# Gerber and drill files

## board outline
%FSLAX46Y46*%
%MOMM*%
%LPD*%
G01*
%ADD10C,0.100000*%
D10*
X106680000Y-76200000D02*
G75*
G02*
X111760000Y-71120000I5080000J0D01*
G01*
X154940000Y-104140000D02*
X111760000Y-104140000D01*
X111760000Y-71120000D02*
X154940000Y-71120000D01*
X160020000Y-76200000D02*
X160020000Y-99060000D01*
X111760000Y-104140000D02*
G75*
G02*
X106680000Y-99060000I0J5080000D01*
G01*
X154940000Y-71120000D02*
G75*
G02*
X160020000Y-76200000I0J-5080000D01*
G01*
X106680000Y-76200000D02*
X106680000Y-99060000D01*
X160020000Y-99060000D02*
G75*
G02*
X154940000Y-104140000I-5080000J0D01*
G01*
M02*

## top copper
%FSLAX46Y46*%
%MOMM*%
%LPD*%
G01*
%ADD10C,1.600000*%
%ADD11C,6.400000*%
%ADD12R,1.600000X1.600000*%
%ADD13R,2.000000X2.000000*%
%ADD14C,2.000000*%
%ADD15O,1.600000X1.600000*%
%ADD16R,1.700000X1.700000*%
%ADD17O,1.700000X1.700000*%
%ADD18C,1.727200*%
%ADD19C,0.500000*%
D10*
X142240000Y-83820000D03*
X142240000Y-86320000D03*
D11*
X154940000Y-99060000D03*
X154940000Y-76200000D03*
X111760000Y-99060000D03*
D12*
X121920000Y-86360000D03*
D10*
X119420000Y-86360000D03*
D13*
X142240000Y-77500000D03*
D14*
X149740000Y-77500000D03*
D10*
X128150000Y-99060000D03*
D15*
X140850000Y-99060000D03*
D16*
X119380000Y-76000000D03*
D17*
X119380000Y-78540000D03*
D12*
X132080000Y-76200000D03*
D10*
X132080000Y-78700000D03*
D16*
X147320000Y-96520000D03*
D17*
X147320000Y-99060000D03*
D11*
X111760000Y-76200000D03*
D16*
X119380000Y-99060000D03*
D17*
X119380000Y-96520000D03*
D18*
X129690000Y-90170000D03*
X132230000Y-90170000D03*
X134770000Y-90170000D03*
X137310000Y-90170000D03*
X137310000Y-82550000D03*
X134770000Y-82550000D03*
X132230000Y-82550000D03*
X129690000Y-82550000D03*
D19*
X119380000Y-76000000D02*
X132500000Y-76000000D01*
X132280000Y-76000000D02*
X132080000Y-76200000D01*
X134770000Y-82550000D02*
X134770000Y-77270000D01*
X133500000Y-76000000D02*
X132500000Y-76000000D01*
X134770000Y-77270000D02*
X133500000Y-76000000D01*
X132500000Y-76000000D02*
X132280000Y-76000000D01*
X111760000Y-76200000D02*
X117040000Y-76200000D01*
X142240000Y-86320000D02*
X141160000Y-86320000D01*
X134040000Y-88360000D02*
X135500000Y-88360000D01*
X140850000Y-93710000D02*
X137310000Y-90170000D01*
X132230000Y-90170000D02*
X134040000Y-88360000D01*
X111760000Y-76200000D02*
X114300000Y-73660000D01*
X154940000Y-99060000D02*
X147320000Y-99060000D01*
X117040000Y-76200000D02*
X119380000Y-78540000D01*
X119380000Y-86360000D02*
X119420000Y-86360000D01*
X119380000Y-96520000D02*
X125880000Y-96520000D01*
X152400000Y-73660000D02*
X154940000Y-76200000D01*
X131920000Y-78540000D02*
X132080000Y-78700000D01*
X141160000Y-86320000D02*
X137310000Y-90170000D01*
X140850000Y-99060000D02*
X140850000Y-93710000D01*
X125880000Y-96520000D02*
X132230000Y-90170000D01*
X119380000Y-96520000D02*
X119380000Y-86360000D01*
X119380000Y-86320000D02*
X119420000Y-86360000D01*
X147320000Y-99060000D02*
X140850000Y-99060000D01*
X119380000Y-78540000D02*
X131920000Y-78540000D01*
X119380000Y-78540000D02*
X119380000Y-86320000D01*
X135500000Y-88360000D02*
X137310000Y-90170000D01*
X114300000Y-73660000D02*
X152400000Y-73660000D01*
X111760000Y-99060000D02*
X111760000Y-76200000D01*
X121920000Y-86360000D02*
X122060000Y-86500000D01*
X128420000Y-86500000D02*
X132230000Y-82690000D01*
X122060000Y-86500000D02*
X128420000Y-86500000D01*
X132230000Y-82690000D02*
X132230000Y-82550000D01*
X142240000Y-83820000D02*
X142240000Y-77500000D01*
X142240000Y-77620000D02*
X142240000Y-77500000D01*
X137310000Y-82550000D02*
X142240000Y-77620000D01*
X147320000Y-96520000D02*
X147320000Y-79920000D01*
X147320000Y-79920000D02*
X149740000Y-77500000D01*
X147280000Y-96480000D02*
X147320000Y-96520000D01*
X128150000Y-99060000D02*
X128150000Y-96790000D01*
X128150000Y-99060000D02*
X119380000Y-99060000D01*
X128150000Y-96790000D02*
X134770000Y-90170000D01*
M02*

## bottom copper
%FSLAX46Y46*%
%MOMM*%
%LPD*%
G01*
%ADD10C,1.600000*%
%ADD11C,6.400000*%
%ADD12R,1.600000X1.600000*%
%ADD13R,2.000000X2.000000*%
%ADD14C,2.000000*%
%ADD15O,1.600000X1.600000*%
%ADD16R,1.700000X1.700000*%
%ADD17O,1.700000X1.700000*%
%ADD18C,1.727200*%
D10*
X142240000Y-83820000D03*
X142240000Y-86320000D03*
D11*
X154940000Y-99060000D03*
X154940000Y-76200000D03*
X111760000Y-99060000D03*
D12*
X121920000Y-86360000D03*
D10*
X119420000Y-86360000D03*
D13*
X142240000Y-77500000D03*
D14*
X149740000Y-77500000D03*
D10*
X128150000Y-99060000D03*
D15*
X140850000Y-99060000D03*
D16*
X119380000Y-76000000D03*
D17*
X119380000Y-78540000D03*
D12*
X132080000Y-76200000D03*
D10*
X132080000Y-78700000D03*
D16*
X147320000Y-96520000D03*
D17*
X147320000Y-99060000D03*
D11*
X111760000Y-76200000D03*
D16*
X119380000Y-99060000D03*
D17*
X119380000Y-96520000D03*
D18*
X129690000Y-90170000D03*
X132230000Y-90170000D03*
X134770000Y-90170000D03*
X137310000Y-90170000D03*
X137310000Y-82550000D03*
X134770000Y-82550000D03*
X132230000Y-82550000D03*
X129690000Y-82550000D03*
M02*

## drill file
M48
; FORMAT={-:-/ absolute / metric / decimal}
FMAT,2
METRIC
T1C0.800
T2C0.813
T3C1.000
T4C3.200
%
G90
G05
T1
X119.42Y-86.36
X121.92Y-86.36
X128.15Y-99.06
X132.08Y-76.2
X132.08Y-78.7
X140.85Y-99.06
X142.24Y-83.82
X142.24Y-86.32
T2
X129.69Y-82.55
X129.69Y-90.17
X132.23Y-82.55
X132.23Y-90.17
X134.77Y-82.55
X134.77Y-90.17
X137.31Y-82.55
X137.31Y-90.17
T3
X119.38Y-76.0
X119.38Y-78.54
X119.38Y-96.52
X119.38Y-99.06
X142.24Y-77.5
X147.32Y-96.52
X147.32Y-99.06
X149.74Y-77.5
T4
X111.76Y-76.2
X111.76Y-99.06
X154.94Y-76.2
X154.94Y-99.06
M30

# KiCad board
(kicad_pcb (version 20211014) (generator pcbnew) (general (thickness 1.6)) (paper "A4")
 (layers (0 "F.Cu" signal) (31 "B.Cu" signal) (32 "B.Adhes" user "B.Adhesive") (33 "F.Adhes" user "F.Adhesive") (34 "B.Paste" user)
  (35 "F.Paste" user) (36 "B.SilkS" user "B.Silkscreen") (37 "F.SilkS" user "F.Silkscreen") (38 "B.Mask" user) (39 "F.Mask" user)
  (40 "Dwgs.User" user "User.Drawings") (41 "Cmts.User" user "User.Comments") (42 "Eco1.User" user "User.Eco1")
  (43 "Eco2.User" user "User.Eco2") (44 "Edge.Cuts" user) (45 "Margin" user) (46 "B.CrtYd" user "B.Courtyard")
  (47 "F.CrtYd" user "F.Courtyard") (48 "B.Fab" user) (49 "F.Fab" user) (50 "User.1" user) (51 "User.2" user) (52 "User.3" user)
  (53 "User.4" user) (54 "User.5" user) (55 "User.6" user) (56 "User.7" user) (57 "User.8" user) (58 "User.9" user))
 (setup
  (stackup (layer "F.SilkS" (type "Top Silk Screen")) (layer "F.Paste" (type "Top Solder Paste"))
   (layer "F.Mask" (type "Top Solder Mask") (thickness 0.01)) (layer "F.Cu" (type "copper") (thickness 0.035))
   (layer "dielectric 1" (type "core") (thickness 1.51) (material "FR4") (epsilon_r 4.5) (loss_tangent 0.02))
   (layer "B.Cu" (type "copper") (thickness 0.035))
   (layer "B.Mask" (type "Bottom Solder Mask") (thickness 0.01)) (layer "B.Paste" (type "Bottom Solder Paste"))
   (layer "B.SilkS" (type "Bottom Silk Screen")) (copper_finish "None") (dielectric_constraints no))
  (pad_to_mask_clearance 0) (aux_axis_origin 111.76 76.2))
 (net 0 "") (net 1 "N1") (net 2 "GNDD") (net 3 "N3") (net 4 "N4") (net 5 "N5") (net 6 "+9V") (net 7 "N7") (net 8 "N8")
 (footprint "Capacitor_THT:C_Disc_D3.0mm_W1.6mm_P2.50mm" (layer "F.Cu") (at 142.24 83.82 -90)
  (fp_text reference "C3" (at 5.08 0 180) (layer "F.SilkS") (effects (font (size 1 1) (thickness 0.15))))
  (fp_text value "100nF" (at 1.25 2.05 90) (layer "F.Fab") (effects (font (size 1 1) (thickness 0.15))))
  (pad "1" thru_hole circle (at 0 0 270) (size 1.6 1.6) (drill 0.8) (layers *.Cu *.Mask) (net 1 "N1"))
  (pad "2" thru_hole circle (at 2.5 0 270) (size 1.6 1.6) (drill 0.8) (layers *.Cu *.Mask) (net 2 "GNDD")))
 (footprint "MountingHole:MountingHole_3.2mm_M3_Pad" (layer "F.Cu") (at 154.94 99.06)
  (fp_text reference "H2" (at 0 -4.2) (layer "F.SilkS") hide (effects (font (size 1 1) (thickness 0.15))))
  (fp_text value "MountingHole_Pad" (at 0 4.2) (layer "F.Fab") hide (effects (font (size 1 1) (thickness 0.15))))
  (pad "1" thru_hole circle (at 0 0) (size 6.4 6.4) (drill 3.2) (layers *.Cu *.Mask) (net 2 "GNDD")))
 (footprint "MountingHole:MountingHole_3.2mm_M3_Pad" (layer "F.Cu") (at 154.94 76.2)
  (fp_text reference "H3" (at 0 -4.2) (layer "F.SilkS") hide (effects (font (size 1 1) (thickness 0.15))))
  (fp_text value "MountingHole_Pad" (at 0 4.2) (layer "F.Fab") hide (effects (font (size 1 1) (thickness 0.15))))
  (pad "1" thru_hole circle (at 0 0) (size 6.4 6.4) (drill 3.2) (layers *.Cu *.Mask) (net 2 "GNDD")))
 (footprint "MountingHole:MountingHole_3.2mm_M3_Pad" (layer "F.Cu") (at 111.76 99.06)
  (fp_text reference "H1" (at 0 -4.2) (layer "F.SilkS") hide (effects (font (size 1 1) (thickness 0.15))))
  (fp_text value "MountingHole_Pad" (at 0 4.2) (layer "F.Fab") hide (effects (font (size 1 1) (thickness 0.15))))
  (pad "1" thru_hole circle (at 0 0) (size 6.4 6.4) (drill 3.2) (layers *.Cu *.Mask) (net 2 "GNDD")))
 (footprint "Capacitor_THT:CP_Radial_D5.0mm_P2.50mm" (layer "F.Cu") (at 121.92 86.36 180)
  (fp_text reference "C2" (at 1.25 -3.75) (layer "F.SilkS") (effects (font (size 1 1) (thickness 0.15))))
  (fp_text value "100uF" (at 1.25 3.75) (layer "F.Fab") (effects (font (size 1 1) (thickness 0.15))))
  (pad "1" thru_hole rect (at 0 0 180) (size 1.6 1.6) (drill 0.8) (layers *.Cu *.Mask) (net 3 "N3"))
  (pad "2" thru_hole circle (at 2.5 0 180) (size 1.6 1.6) (drill 0.8) (layers *.Cu *.Mask) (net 2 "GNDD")))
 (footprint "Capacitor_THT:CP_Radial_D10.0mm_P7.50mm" (layer "F.Cu") (at 142.24 77.5)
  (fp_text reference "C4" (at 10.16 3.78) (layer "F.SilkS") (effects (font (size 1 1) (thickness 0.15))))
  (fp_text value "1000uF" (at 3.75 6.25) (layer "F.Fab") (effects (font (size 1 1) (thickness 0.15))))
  (pad "1" thru_hole rect (at 0 0) (size 2 2) (drill 1) (layers *.Cu *.Mask) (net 1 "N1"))
  (pad "2" thru_hole circle (at 7.5 0) (size 2 2) (drill 1) (layers *.Cu *.Mask) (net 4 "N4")))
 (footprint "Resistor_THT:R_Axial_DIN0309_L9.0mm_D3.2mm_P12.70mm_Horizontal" (layer "F.Cu") (at 128.15 99.06)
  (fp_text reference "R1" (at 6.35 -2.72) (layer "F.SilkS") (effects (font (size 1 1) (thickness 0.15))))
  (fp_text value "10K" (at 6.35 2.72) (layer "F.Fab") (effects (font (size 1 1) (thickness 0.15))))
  (pad "1" thru_hole circle (at 0 0) (size 1.6 1.6) (drill 0.8) (layers *.Cu *.Mask) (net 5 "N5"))
  (pad "2" thru_hole oval (at 12.7 0) (size 1.6 1.6) (drill 0.8) (layers *.Cu *.Mask) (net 2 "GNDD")))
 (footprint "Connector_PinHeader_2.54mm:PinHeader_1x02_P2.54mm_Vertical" (layer "F.Cu") (at 119.38 76)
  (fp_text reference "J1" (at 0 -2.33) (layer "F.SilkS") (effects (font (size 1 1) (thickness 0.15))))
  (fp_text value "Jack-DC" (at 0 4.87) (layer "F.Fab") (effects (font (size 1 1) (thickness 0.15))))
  (pad "1" thru_hole rect (at 0 0) (size 1.7 1.7) (drill 1) (layers *.Cu *.Mask) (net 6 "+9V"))
  (pad "2" thru_hole oval (at 0 2.54) (size 1.7 1.7) (drill 1) (layers *.Cu *.Mask) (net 2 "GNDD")))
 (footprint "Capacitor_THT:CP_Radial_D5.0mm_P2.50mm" (layer "F.Cu") (at 132.08 76.2 -90)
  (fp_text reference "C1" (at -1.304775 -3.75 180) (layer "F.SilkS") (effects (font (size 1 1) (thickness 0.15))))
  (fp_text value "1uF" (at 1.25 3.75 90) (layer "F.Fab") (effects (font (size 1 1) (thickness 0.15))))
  (pad "1" thru_hole rect (at 0 0 270) (size 1.6 1.6) (drill 0.8) (layers *.Cu *.Mask) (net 6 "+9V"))
  (pad "2" thru_hole circle (at 2.5 0 270) (size 1.6 1.6) (drill 0.8) (layers *.Cu *.Mask) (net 2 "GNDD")))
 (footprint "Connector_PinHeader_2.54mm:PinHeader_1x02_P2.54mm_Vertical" (layer "F.Cu") (at 147.32 96.52)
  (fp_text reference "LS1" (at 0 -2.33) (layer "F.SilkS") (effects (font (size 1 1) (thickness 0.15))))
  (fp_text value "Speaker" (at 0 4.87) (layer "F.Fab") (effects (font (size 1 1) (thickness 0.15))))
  (pad "1" thru_hole rect (at 0 0) (size 1.7 1.7) (drill 1) (layers *.Cu *.Mask) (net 4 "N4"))
  (pad "2" thru_hole oval (at 0 2.54) (size 1.7 1.7) (drill 1) (layers *.Cu *.Mask) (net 2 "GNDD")))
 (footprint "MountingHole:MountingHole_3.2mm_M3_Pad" (layer "F.Cu") (at 111.76 76.2)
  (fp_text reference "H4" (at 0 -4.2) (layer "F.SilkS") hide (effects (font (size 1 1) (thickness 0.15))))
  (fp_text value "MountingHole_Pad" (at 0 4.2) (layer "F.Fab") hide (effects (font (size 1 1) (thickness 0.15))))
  (pad "1" thru_hole circle (at 0 0) (size 6.4 6.4) (drill 3.2) (layers *.Cu *.Mask) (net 2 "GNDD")))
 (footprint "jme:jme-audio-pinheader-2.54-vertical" (layer "F.Cu") (at 119.38 99.06 180)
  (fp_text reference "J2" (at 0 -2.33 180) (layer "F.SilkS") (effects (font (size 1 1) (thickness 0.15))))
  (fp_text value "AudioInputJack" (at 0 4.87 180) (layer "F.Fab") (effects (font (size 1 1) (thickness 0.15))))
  (pad "1" thru_hole rect (at 0 0 180) (size 1.7 1.7) (drill 1) (layers *.Cu *.Mask))
  (pad "2" thru_hole oval (at 0 2.54 180) (size 1.7 1.7) (drill 1) (layers *.Cu *.Mask)))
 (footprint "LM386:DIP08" (layer "F.Cu") (at 133.5 86.36)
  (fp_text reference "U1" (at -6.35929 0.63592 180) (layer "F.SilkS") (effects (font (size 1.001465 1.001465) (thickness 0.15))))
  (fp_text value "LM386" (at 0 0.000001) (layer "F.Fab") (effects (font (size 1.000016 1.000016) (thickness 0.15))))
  (pad "1" thru_hole circle locked (at -3.81 3.81) (size 1.7272 1.7272) (drill 0.8128) (layers *.Cu *.Mask) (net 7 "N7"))
  (pad "2" thru_hole circle locked (at -1.27 3.81) (size 1.7272 1.7272) (drill 0.8128) (layers *.Cu *.Mask) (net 2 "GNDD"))
  (pad "3" thru_hole circle locked (at 1.27 3.81) (size 1.7272 1.7272) (drill 0.8128) (layers *.Cu *.Mask) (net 5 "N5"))
  (pad "4" thru_hole circle locked (at 3.81 3.81) (size 1.7272 1.7272) (drill 0.8128) (layers *.Cu *.Mask) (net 2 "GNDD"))
  (pad "5" thru_hole circle locked (at 3.81 -3.81) (size 1.7272 1.7272) (drill 0.8128) (layers *.Cu *.Mask) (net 1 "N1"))
  (pad "6" thru_hole circle locked (at 1.27 -3.81) (size 1.7272 1.7272) (drill 0.8128) (layers *.Cu *.Mask) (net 6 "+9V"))
  (pad "7" thru_hole circle locked (at -1.27 -3.81) (size 1.7272 1.7272) (drill 0.8128) (layers *.Cu *.Mask) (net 3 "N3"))
  (pad "8" thru_hole circle locked (at -3.81 -3.81) (size 1.7272 1.7272) (drill 0.8128) (layers *.Cu *.Mask) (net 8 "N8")))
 (gr_arc (start 106.68 76.2) (mid 108.167898 72.607898) (end 111.76 71.12) (layer "Edge.Cuts") (width 0.1))
 (gr_line (start 154.94 104.14) (end 111.76 104.14) (layer "Edge.Cuts") (width 0.1))
 (gr_line (start 111.76 71.12) (end 154.94 71.12) (layer "Edge.Cuts") (width 0.1))
 (gr_line (start 160.02 76.2) (end 160.02 99.06) (layer "Edge.Cuts") (width 0.1))
 (gr_arc (start 111.76 104.14) (mid 108.167898 102.652102) (end 106.68 99.06) (layer "Edge.Cuts") (width 0.1))
 (gr_arc (start 154.94 71.12) (mid 158.532102 72.607898) (end 160.02 76.2) (layer "Edge.Cuts") (width 0.1))
 (gr_line (start 106.68 76.2) (end 106.68 99.06) (layer "Edge.Cuts") (width 0.1))
 (gr_arc (start 160.02 99.06) (mid 158.532102 102.652102) (end 154.94 104.14) (layer "Edge.Cuts") (width 0.1))
 (segment (start 119.38 76) (end 132.5 76) (width 0.5) (layer "F.Cu") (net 6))
 (segment (start 132.28 76) (end 132.08 76.2) (width 0.5) (layer "F.Cu") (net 6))
 (segment (start 134.77 82.55) (end 134.77 77.27) (width 0.5) (layer "F.Cu") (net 6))
 (segment (start 133.5 76) (end 132.5 76) (width 0.5) (layer "F.Cu") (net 6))
 (segment (start 134.77 77.27) (end 133.5 76) (width 0.5) (layer "F.Cu") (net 6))
 (segment (start 132.5 76) (end 132.28 76) (width 0.5) (layer "F.Cu") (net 6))
 (segment (start 111.76 76.2) (end 117.04 76.2) (width 0.5) (layer "F.Cu") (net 2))
 (segment (start 142.24 86.32) (end 141.16 86.32) (width 0.5) (layer "F.Cu") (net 2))
 (segment (start 134.04 88.36) (end 135.5 88.36) (width 0.5) (layer "F.Cu") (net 2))
 (segment (start 140.85 93.71) (end 137.31 90.17) (width 0.5) (layer "F.Cu") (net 2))
 (segment (start 132.23 90.17) (end 134.04 88.36) (width 0.5) (layer "F.Cu") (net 2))
 (segment (start 111.76 76.2) (end 114.3 73.66) (width 0.5) (layer "F.Cu") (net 2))
 (segment (start 154.94 99.06) (end 147.32 99.06) (width 0.5) (layer "F.Cu") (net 2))
 (segment (start 117.04 76.2) (end 119.38 78.54) (width 0.5) (layer "F.Cu") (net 2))
 (segment (start 119.38 86.36) (end 119.42 86.36) (width 0.5) (layer "F.Cu") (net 2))
 (segment (start 119.38 96.52) (end 125.88 96.52) (width 0.5) (layer "F.Cu") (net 2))
 (segment (start 152.4 73.66) (end 154.94 76.2) (width 0.5) (layer "F.Cu") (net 2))
 (segment (start 131.92 78.54) (end 132.08 78.7) (width 0.5) (layer "F.Cu") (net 2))
 (segment (start 141.16 86.32) (end 137.31 90.17) (width 0.5) (layer "F.Cu") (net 2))
 (segment (start 140.85 99.06) (end 140.85 93.71) (width 0.5) (layer "F.Cu") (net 2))
 (segment (start 125.88 96.52) (end 132.23 90.17) (width 0.5) (layer "F.Cu") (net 2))
 (segment (start 119.38 96.52) (end 119.38 86.36) (width 0.5) (layer "F.Cu") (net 2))
 (segment (start 119.38 86.32) (end 119.42 86.36) (width 0.5) (layer "F.Cu") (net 2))
 (segment (start 147.32 99.06) (end 140.85 99.06) (width 0.5) (layer "F.Cu") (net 2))
 (segment (start 119.38 78.54) (end 131.92 78.54) (width 0.5) (layer "F.Cu") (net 2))
 (segment (start 119.38 78.54) (end 119.38 86.32) (width 0.5) (layer "F.Cu") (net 2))
 (segment (start 135.5 88.36) (end 137.31 90.17) (width 0.5) (layer "F.Cu") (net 2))
 (segment (start 114.3 73.66) (end 152.4 73.66) (width 0.5) (layer "F.Cu") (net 2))
 (segment (start 111.76 99.06) (end 111.76 76.2) (width 0.5) (layer "F.Cu") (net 2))
 (segment (start 121.92 86.36) (end 122.06 86.5) (width 0.5) (layer "F.Cu") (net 3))
 (segment (start 128.42 86.5) (end 132.23 82.69) (width 0.5) (layer "F.Cu") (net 3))
 (segment (start 122.06 86.5) (end 128.42 86.5) (width 0.5) (layer "F.Cu") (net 3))
 (segment (start 132.23 82.69) (end 132.23 82.55) (width 0.5) (layer "F.Cu") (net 3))
 (segment (start 142.24 83.82) (end 142.24 77.5) (width 0.5) (layer "F.Cu") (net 1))
 (segment (start 142.24 77.62) (end 142.24 77.5) (width 0.5) (layer "F.Cu") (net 1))
 (segment (start 137.31 82.55) (end 142.24 77.62) (width 0.5) (layer "F.Cu") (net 1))
 (segment (start 147.32 96.52) (end 147.32 79.92) (width 0.5) (layer "F.Cu") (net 4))
 (segment (start 147.32 79.92) (end 149.74 77.5) (width 0.5) (layer "F.Cu") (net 4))
 (segment (start 147.28 96.48) (end 147.32 96.52) (width 0.5) (layer "F.Cu") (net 4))
 (segment (start 128.15 99.06) (end 128.15 96.79) (width 0.5) (layer "F.Cu") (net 5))
 (segment (start 128.15 99.06) (end 119.38 99.06) (width 0.5) (layer "F.Cu") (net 5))
 (segment (start 128.15 96.79) (end 134.77 90.17) (width 0.5) (layer "F.Cu") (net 5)))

